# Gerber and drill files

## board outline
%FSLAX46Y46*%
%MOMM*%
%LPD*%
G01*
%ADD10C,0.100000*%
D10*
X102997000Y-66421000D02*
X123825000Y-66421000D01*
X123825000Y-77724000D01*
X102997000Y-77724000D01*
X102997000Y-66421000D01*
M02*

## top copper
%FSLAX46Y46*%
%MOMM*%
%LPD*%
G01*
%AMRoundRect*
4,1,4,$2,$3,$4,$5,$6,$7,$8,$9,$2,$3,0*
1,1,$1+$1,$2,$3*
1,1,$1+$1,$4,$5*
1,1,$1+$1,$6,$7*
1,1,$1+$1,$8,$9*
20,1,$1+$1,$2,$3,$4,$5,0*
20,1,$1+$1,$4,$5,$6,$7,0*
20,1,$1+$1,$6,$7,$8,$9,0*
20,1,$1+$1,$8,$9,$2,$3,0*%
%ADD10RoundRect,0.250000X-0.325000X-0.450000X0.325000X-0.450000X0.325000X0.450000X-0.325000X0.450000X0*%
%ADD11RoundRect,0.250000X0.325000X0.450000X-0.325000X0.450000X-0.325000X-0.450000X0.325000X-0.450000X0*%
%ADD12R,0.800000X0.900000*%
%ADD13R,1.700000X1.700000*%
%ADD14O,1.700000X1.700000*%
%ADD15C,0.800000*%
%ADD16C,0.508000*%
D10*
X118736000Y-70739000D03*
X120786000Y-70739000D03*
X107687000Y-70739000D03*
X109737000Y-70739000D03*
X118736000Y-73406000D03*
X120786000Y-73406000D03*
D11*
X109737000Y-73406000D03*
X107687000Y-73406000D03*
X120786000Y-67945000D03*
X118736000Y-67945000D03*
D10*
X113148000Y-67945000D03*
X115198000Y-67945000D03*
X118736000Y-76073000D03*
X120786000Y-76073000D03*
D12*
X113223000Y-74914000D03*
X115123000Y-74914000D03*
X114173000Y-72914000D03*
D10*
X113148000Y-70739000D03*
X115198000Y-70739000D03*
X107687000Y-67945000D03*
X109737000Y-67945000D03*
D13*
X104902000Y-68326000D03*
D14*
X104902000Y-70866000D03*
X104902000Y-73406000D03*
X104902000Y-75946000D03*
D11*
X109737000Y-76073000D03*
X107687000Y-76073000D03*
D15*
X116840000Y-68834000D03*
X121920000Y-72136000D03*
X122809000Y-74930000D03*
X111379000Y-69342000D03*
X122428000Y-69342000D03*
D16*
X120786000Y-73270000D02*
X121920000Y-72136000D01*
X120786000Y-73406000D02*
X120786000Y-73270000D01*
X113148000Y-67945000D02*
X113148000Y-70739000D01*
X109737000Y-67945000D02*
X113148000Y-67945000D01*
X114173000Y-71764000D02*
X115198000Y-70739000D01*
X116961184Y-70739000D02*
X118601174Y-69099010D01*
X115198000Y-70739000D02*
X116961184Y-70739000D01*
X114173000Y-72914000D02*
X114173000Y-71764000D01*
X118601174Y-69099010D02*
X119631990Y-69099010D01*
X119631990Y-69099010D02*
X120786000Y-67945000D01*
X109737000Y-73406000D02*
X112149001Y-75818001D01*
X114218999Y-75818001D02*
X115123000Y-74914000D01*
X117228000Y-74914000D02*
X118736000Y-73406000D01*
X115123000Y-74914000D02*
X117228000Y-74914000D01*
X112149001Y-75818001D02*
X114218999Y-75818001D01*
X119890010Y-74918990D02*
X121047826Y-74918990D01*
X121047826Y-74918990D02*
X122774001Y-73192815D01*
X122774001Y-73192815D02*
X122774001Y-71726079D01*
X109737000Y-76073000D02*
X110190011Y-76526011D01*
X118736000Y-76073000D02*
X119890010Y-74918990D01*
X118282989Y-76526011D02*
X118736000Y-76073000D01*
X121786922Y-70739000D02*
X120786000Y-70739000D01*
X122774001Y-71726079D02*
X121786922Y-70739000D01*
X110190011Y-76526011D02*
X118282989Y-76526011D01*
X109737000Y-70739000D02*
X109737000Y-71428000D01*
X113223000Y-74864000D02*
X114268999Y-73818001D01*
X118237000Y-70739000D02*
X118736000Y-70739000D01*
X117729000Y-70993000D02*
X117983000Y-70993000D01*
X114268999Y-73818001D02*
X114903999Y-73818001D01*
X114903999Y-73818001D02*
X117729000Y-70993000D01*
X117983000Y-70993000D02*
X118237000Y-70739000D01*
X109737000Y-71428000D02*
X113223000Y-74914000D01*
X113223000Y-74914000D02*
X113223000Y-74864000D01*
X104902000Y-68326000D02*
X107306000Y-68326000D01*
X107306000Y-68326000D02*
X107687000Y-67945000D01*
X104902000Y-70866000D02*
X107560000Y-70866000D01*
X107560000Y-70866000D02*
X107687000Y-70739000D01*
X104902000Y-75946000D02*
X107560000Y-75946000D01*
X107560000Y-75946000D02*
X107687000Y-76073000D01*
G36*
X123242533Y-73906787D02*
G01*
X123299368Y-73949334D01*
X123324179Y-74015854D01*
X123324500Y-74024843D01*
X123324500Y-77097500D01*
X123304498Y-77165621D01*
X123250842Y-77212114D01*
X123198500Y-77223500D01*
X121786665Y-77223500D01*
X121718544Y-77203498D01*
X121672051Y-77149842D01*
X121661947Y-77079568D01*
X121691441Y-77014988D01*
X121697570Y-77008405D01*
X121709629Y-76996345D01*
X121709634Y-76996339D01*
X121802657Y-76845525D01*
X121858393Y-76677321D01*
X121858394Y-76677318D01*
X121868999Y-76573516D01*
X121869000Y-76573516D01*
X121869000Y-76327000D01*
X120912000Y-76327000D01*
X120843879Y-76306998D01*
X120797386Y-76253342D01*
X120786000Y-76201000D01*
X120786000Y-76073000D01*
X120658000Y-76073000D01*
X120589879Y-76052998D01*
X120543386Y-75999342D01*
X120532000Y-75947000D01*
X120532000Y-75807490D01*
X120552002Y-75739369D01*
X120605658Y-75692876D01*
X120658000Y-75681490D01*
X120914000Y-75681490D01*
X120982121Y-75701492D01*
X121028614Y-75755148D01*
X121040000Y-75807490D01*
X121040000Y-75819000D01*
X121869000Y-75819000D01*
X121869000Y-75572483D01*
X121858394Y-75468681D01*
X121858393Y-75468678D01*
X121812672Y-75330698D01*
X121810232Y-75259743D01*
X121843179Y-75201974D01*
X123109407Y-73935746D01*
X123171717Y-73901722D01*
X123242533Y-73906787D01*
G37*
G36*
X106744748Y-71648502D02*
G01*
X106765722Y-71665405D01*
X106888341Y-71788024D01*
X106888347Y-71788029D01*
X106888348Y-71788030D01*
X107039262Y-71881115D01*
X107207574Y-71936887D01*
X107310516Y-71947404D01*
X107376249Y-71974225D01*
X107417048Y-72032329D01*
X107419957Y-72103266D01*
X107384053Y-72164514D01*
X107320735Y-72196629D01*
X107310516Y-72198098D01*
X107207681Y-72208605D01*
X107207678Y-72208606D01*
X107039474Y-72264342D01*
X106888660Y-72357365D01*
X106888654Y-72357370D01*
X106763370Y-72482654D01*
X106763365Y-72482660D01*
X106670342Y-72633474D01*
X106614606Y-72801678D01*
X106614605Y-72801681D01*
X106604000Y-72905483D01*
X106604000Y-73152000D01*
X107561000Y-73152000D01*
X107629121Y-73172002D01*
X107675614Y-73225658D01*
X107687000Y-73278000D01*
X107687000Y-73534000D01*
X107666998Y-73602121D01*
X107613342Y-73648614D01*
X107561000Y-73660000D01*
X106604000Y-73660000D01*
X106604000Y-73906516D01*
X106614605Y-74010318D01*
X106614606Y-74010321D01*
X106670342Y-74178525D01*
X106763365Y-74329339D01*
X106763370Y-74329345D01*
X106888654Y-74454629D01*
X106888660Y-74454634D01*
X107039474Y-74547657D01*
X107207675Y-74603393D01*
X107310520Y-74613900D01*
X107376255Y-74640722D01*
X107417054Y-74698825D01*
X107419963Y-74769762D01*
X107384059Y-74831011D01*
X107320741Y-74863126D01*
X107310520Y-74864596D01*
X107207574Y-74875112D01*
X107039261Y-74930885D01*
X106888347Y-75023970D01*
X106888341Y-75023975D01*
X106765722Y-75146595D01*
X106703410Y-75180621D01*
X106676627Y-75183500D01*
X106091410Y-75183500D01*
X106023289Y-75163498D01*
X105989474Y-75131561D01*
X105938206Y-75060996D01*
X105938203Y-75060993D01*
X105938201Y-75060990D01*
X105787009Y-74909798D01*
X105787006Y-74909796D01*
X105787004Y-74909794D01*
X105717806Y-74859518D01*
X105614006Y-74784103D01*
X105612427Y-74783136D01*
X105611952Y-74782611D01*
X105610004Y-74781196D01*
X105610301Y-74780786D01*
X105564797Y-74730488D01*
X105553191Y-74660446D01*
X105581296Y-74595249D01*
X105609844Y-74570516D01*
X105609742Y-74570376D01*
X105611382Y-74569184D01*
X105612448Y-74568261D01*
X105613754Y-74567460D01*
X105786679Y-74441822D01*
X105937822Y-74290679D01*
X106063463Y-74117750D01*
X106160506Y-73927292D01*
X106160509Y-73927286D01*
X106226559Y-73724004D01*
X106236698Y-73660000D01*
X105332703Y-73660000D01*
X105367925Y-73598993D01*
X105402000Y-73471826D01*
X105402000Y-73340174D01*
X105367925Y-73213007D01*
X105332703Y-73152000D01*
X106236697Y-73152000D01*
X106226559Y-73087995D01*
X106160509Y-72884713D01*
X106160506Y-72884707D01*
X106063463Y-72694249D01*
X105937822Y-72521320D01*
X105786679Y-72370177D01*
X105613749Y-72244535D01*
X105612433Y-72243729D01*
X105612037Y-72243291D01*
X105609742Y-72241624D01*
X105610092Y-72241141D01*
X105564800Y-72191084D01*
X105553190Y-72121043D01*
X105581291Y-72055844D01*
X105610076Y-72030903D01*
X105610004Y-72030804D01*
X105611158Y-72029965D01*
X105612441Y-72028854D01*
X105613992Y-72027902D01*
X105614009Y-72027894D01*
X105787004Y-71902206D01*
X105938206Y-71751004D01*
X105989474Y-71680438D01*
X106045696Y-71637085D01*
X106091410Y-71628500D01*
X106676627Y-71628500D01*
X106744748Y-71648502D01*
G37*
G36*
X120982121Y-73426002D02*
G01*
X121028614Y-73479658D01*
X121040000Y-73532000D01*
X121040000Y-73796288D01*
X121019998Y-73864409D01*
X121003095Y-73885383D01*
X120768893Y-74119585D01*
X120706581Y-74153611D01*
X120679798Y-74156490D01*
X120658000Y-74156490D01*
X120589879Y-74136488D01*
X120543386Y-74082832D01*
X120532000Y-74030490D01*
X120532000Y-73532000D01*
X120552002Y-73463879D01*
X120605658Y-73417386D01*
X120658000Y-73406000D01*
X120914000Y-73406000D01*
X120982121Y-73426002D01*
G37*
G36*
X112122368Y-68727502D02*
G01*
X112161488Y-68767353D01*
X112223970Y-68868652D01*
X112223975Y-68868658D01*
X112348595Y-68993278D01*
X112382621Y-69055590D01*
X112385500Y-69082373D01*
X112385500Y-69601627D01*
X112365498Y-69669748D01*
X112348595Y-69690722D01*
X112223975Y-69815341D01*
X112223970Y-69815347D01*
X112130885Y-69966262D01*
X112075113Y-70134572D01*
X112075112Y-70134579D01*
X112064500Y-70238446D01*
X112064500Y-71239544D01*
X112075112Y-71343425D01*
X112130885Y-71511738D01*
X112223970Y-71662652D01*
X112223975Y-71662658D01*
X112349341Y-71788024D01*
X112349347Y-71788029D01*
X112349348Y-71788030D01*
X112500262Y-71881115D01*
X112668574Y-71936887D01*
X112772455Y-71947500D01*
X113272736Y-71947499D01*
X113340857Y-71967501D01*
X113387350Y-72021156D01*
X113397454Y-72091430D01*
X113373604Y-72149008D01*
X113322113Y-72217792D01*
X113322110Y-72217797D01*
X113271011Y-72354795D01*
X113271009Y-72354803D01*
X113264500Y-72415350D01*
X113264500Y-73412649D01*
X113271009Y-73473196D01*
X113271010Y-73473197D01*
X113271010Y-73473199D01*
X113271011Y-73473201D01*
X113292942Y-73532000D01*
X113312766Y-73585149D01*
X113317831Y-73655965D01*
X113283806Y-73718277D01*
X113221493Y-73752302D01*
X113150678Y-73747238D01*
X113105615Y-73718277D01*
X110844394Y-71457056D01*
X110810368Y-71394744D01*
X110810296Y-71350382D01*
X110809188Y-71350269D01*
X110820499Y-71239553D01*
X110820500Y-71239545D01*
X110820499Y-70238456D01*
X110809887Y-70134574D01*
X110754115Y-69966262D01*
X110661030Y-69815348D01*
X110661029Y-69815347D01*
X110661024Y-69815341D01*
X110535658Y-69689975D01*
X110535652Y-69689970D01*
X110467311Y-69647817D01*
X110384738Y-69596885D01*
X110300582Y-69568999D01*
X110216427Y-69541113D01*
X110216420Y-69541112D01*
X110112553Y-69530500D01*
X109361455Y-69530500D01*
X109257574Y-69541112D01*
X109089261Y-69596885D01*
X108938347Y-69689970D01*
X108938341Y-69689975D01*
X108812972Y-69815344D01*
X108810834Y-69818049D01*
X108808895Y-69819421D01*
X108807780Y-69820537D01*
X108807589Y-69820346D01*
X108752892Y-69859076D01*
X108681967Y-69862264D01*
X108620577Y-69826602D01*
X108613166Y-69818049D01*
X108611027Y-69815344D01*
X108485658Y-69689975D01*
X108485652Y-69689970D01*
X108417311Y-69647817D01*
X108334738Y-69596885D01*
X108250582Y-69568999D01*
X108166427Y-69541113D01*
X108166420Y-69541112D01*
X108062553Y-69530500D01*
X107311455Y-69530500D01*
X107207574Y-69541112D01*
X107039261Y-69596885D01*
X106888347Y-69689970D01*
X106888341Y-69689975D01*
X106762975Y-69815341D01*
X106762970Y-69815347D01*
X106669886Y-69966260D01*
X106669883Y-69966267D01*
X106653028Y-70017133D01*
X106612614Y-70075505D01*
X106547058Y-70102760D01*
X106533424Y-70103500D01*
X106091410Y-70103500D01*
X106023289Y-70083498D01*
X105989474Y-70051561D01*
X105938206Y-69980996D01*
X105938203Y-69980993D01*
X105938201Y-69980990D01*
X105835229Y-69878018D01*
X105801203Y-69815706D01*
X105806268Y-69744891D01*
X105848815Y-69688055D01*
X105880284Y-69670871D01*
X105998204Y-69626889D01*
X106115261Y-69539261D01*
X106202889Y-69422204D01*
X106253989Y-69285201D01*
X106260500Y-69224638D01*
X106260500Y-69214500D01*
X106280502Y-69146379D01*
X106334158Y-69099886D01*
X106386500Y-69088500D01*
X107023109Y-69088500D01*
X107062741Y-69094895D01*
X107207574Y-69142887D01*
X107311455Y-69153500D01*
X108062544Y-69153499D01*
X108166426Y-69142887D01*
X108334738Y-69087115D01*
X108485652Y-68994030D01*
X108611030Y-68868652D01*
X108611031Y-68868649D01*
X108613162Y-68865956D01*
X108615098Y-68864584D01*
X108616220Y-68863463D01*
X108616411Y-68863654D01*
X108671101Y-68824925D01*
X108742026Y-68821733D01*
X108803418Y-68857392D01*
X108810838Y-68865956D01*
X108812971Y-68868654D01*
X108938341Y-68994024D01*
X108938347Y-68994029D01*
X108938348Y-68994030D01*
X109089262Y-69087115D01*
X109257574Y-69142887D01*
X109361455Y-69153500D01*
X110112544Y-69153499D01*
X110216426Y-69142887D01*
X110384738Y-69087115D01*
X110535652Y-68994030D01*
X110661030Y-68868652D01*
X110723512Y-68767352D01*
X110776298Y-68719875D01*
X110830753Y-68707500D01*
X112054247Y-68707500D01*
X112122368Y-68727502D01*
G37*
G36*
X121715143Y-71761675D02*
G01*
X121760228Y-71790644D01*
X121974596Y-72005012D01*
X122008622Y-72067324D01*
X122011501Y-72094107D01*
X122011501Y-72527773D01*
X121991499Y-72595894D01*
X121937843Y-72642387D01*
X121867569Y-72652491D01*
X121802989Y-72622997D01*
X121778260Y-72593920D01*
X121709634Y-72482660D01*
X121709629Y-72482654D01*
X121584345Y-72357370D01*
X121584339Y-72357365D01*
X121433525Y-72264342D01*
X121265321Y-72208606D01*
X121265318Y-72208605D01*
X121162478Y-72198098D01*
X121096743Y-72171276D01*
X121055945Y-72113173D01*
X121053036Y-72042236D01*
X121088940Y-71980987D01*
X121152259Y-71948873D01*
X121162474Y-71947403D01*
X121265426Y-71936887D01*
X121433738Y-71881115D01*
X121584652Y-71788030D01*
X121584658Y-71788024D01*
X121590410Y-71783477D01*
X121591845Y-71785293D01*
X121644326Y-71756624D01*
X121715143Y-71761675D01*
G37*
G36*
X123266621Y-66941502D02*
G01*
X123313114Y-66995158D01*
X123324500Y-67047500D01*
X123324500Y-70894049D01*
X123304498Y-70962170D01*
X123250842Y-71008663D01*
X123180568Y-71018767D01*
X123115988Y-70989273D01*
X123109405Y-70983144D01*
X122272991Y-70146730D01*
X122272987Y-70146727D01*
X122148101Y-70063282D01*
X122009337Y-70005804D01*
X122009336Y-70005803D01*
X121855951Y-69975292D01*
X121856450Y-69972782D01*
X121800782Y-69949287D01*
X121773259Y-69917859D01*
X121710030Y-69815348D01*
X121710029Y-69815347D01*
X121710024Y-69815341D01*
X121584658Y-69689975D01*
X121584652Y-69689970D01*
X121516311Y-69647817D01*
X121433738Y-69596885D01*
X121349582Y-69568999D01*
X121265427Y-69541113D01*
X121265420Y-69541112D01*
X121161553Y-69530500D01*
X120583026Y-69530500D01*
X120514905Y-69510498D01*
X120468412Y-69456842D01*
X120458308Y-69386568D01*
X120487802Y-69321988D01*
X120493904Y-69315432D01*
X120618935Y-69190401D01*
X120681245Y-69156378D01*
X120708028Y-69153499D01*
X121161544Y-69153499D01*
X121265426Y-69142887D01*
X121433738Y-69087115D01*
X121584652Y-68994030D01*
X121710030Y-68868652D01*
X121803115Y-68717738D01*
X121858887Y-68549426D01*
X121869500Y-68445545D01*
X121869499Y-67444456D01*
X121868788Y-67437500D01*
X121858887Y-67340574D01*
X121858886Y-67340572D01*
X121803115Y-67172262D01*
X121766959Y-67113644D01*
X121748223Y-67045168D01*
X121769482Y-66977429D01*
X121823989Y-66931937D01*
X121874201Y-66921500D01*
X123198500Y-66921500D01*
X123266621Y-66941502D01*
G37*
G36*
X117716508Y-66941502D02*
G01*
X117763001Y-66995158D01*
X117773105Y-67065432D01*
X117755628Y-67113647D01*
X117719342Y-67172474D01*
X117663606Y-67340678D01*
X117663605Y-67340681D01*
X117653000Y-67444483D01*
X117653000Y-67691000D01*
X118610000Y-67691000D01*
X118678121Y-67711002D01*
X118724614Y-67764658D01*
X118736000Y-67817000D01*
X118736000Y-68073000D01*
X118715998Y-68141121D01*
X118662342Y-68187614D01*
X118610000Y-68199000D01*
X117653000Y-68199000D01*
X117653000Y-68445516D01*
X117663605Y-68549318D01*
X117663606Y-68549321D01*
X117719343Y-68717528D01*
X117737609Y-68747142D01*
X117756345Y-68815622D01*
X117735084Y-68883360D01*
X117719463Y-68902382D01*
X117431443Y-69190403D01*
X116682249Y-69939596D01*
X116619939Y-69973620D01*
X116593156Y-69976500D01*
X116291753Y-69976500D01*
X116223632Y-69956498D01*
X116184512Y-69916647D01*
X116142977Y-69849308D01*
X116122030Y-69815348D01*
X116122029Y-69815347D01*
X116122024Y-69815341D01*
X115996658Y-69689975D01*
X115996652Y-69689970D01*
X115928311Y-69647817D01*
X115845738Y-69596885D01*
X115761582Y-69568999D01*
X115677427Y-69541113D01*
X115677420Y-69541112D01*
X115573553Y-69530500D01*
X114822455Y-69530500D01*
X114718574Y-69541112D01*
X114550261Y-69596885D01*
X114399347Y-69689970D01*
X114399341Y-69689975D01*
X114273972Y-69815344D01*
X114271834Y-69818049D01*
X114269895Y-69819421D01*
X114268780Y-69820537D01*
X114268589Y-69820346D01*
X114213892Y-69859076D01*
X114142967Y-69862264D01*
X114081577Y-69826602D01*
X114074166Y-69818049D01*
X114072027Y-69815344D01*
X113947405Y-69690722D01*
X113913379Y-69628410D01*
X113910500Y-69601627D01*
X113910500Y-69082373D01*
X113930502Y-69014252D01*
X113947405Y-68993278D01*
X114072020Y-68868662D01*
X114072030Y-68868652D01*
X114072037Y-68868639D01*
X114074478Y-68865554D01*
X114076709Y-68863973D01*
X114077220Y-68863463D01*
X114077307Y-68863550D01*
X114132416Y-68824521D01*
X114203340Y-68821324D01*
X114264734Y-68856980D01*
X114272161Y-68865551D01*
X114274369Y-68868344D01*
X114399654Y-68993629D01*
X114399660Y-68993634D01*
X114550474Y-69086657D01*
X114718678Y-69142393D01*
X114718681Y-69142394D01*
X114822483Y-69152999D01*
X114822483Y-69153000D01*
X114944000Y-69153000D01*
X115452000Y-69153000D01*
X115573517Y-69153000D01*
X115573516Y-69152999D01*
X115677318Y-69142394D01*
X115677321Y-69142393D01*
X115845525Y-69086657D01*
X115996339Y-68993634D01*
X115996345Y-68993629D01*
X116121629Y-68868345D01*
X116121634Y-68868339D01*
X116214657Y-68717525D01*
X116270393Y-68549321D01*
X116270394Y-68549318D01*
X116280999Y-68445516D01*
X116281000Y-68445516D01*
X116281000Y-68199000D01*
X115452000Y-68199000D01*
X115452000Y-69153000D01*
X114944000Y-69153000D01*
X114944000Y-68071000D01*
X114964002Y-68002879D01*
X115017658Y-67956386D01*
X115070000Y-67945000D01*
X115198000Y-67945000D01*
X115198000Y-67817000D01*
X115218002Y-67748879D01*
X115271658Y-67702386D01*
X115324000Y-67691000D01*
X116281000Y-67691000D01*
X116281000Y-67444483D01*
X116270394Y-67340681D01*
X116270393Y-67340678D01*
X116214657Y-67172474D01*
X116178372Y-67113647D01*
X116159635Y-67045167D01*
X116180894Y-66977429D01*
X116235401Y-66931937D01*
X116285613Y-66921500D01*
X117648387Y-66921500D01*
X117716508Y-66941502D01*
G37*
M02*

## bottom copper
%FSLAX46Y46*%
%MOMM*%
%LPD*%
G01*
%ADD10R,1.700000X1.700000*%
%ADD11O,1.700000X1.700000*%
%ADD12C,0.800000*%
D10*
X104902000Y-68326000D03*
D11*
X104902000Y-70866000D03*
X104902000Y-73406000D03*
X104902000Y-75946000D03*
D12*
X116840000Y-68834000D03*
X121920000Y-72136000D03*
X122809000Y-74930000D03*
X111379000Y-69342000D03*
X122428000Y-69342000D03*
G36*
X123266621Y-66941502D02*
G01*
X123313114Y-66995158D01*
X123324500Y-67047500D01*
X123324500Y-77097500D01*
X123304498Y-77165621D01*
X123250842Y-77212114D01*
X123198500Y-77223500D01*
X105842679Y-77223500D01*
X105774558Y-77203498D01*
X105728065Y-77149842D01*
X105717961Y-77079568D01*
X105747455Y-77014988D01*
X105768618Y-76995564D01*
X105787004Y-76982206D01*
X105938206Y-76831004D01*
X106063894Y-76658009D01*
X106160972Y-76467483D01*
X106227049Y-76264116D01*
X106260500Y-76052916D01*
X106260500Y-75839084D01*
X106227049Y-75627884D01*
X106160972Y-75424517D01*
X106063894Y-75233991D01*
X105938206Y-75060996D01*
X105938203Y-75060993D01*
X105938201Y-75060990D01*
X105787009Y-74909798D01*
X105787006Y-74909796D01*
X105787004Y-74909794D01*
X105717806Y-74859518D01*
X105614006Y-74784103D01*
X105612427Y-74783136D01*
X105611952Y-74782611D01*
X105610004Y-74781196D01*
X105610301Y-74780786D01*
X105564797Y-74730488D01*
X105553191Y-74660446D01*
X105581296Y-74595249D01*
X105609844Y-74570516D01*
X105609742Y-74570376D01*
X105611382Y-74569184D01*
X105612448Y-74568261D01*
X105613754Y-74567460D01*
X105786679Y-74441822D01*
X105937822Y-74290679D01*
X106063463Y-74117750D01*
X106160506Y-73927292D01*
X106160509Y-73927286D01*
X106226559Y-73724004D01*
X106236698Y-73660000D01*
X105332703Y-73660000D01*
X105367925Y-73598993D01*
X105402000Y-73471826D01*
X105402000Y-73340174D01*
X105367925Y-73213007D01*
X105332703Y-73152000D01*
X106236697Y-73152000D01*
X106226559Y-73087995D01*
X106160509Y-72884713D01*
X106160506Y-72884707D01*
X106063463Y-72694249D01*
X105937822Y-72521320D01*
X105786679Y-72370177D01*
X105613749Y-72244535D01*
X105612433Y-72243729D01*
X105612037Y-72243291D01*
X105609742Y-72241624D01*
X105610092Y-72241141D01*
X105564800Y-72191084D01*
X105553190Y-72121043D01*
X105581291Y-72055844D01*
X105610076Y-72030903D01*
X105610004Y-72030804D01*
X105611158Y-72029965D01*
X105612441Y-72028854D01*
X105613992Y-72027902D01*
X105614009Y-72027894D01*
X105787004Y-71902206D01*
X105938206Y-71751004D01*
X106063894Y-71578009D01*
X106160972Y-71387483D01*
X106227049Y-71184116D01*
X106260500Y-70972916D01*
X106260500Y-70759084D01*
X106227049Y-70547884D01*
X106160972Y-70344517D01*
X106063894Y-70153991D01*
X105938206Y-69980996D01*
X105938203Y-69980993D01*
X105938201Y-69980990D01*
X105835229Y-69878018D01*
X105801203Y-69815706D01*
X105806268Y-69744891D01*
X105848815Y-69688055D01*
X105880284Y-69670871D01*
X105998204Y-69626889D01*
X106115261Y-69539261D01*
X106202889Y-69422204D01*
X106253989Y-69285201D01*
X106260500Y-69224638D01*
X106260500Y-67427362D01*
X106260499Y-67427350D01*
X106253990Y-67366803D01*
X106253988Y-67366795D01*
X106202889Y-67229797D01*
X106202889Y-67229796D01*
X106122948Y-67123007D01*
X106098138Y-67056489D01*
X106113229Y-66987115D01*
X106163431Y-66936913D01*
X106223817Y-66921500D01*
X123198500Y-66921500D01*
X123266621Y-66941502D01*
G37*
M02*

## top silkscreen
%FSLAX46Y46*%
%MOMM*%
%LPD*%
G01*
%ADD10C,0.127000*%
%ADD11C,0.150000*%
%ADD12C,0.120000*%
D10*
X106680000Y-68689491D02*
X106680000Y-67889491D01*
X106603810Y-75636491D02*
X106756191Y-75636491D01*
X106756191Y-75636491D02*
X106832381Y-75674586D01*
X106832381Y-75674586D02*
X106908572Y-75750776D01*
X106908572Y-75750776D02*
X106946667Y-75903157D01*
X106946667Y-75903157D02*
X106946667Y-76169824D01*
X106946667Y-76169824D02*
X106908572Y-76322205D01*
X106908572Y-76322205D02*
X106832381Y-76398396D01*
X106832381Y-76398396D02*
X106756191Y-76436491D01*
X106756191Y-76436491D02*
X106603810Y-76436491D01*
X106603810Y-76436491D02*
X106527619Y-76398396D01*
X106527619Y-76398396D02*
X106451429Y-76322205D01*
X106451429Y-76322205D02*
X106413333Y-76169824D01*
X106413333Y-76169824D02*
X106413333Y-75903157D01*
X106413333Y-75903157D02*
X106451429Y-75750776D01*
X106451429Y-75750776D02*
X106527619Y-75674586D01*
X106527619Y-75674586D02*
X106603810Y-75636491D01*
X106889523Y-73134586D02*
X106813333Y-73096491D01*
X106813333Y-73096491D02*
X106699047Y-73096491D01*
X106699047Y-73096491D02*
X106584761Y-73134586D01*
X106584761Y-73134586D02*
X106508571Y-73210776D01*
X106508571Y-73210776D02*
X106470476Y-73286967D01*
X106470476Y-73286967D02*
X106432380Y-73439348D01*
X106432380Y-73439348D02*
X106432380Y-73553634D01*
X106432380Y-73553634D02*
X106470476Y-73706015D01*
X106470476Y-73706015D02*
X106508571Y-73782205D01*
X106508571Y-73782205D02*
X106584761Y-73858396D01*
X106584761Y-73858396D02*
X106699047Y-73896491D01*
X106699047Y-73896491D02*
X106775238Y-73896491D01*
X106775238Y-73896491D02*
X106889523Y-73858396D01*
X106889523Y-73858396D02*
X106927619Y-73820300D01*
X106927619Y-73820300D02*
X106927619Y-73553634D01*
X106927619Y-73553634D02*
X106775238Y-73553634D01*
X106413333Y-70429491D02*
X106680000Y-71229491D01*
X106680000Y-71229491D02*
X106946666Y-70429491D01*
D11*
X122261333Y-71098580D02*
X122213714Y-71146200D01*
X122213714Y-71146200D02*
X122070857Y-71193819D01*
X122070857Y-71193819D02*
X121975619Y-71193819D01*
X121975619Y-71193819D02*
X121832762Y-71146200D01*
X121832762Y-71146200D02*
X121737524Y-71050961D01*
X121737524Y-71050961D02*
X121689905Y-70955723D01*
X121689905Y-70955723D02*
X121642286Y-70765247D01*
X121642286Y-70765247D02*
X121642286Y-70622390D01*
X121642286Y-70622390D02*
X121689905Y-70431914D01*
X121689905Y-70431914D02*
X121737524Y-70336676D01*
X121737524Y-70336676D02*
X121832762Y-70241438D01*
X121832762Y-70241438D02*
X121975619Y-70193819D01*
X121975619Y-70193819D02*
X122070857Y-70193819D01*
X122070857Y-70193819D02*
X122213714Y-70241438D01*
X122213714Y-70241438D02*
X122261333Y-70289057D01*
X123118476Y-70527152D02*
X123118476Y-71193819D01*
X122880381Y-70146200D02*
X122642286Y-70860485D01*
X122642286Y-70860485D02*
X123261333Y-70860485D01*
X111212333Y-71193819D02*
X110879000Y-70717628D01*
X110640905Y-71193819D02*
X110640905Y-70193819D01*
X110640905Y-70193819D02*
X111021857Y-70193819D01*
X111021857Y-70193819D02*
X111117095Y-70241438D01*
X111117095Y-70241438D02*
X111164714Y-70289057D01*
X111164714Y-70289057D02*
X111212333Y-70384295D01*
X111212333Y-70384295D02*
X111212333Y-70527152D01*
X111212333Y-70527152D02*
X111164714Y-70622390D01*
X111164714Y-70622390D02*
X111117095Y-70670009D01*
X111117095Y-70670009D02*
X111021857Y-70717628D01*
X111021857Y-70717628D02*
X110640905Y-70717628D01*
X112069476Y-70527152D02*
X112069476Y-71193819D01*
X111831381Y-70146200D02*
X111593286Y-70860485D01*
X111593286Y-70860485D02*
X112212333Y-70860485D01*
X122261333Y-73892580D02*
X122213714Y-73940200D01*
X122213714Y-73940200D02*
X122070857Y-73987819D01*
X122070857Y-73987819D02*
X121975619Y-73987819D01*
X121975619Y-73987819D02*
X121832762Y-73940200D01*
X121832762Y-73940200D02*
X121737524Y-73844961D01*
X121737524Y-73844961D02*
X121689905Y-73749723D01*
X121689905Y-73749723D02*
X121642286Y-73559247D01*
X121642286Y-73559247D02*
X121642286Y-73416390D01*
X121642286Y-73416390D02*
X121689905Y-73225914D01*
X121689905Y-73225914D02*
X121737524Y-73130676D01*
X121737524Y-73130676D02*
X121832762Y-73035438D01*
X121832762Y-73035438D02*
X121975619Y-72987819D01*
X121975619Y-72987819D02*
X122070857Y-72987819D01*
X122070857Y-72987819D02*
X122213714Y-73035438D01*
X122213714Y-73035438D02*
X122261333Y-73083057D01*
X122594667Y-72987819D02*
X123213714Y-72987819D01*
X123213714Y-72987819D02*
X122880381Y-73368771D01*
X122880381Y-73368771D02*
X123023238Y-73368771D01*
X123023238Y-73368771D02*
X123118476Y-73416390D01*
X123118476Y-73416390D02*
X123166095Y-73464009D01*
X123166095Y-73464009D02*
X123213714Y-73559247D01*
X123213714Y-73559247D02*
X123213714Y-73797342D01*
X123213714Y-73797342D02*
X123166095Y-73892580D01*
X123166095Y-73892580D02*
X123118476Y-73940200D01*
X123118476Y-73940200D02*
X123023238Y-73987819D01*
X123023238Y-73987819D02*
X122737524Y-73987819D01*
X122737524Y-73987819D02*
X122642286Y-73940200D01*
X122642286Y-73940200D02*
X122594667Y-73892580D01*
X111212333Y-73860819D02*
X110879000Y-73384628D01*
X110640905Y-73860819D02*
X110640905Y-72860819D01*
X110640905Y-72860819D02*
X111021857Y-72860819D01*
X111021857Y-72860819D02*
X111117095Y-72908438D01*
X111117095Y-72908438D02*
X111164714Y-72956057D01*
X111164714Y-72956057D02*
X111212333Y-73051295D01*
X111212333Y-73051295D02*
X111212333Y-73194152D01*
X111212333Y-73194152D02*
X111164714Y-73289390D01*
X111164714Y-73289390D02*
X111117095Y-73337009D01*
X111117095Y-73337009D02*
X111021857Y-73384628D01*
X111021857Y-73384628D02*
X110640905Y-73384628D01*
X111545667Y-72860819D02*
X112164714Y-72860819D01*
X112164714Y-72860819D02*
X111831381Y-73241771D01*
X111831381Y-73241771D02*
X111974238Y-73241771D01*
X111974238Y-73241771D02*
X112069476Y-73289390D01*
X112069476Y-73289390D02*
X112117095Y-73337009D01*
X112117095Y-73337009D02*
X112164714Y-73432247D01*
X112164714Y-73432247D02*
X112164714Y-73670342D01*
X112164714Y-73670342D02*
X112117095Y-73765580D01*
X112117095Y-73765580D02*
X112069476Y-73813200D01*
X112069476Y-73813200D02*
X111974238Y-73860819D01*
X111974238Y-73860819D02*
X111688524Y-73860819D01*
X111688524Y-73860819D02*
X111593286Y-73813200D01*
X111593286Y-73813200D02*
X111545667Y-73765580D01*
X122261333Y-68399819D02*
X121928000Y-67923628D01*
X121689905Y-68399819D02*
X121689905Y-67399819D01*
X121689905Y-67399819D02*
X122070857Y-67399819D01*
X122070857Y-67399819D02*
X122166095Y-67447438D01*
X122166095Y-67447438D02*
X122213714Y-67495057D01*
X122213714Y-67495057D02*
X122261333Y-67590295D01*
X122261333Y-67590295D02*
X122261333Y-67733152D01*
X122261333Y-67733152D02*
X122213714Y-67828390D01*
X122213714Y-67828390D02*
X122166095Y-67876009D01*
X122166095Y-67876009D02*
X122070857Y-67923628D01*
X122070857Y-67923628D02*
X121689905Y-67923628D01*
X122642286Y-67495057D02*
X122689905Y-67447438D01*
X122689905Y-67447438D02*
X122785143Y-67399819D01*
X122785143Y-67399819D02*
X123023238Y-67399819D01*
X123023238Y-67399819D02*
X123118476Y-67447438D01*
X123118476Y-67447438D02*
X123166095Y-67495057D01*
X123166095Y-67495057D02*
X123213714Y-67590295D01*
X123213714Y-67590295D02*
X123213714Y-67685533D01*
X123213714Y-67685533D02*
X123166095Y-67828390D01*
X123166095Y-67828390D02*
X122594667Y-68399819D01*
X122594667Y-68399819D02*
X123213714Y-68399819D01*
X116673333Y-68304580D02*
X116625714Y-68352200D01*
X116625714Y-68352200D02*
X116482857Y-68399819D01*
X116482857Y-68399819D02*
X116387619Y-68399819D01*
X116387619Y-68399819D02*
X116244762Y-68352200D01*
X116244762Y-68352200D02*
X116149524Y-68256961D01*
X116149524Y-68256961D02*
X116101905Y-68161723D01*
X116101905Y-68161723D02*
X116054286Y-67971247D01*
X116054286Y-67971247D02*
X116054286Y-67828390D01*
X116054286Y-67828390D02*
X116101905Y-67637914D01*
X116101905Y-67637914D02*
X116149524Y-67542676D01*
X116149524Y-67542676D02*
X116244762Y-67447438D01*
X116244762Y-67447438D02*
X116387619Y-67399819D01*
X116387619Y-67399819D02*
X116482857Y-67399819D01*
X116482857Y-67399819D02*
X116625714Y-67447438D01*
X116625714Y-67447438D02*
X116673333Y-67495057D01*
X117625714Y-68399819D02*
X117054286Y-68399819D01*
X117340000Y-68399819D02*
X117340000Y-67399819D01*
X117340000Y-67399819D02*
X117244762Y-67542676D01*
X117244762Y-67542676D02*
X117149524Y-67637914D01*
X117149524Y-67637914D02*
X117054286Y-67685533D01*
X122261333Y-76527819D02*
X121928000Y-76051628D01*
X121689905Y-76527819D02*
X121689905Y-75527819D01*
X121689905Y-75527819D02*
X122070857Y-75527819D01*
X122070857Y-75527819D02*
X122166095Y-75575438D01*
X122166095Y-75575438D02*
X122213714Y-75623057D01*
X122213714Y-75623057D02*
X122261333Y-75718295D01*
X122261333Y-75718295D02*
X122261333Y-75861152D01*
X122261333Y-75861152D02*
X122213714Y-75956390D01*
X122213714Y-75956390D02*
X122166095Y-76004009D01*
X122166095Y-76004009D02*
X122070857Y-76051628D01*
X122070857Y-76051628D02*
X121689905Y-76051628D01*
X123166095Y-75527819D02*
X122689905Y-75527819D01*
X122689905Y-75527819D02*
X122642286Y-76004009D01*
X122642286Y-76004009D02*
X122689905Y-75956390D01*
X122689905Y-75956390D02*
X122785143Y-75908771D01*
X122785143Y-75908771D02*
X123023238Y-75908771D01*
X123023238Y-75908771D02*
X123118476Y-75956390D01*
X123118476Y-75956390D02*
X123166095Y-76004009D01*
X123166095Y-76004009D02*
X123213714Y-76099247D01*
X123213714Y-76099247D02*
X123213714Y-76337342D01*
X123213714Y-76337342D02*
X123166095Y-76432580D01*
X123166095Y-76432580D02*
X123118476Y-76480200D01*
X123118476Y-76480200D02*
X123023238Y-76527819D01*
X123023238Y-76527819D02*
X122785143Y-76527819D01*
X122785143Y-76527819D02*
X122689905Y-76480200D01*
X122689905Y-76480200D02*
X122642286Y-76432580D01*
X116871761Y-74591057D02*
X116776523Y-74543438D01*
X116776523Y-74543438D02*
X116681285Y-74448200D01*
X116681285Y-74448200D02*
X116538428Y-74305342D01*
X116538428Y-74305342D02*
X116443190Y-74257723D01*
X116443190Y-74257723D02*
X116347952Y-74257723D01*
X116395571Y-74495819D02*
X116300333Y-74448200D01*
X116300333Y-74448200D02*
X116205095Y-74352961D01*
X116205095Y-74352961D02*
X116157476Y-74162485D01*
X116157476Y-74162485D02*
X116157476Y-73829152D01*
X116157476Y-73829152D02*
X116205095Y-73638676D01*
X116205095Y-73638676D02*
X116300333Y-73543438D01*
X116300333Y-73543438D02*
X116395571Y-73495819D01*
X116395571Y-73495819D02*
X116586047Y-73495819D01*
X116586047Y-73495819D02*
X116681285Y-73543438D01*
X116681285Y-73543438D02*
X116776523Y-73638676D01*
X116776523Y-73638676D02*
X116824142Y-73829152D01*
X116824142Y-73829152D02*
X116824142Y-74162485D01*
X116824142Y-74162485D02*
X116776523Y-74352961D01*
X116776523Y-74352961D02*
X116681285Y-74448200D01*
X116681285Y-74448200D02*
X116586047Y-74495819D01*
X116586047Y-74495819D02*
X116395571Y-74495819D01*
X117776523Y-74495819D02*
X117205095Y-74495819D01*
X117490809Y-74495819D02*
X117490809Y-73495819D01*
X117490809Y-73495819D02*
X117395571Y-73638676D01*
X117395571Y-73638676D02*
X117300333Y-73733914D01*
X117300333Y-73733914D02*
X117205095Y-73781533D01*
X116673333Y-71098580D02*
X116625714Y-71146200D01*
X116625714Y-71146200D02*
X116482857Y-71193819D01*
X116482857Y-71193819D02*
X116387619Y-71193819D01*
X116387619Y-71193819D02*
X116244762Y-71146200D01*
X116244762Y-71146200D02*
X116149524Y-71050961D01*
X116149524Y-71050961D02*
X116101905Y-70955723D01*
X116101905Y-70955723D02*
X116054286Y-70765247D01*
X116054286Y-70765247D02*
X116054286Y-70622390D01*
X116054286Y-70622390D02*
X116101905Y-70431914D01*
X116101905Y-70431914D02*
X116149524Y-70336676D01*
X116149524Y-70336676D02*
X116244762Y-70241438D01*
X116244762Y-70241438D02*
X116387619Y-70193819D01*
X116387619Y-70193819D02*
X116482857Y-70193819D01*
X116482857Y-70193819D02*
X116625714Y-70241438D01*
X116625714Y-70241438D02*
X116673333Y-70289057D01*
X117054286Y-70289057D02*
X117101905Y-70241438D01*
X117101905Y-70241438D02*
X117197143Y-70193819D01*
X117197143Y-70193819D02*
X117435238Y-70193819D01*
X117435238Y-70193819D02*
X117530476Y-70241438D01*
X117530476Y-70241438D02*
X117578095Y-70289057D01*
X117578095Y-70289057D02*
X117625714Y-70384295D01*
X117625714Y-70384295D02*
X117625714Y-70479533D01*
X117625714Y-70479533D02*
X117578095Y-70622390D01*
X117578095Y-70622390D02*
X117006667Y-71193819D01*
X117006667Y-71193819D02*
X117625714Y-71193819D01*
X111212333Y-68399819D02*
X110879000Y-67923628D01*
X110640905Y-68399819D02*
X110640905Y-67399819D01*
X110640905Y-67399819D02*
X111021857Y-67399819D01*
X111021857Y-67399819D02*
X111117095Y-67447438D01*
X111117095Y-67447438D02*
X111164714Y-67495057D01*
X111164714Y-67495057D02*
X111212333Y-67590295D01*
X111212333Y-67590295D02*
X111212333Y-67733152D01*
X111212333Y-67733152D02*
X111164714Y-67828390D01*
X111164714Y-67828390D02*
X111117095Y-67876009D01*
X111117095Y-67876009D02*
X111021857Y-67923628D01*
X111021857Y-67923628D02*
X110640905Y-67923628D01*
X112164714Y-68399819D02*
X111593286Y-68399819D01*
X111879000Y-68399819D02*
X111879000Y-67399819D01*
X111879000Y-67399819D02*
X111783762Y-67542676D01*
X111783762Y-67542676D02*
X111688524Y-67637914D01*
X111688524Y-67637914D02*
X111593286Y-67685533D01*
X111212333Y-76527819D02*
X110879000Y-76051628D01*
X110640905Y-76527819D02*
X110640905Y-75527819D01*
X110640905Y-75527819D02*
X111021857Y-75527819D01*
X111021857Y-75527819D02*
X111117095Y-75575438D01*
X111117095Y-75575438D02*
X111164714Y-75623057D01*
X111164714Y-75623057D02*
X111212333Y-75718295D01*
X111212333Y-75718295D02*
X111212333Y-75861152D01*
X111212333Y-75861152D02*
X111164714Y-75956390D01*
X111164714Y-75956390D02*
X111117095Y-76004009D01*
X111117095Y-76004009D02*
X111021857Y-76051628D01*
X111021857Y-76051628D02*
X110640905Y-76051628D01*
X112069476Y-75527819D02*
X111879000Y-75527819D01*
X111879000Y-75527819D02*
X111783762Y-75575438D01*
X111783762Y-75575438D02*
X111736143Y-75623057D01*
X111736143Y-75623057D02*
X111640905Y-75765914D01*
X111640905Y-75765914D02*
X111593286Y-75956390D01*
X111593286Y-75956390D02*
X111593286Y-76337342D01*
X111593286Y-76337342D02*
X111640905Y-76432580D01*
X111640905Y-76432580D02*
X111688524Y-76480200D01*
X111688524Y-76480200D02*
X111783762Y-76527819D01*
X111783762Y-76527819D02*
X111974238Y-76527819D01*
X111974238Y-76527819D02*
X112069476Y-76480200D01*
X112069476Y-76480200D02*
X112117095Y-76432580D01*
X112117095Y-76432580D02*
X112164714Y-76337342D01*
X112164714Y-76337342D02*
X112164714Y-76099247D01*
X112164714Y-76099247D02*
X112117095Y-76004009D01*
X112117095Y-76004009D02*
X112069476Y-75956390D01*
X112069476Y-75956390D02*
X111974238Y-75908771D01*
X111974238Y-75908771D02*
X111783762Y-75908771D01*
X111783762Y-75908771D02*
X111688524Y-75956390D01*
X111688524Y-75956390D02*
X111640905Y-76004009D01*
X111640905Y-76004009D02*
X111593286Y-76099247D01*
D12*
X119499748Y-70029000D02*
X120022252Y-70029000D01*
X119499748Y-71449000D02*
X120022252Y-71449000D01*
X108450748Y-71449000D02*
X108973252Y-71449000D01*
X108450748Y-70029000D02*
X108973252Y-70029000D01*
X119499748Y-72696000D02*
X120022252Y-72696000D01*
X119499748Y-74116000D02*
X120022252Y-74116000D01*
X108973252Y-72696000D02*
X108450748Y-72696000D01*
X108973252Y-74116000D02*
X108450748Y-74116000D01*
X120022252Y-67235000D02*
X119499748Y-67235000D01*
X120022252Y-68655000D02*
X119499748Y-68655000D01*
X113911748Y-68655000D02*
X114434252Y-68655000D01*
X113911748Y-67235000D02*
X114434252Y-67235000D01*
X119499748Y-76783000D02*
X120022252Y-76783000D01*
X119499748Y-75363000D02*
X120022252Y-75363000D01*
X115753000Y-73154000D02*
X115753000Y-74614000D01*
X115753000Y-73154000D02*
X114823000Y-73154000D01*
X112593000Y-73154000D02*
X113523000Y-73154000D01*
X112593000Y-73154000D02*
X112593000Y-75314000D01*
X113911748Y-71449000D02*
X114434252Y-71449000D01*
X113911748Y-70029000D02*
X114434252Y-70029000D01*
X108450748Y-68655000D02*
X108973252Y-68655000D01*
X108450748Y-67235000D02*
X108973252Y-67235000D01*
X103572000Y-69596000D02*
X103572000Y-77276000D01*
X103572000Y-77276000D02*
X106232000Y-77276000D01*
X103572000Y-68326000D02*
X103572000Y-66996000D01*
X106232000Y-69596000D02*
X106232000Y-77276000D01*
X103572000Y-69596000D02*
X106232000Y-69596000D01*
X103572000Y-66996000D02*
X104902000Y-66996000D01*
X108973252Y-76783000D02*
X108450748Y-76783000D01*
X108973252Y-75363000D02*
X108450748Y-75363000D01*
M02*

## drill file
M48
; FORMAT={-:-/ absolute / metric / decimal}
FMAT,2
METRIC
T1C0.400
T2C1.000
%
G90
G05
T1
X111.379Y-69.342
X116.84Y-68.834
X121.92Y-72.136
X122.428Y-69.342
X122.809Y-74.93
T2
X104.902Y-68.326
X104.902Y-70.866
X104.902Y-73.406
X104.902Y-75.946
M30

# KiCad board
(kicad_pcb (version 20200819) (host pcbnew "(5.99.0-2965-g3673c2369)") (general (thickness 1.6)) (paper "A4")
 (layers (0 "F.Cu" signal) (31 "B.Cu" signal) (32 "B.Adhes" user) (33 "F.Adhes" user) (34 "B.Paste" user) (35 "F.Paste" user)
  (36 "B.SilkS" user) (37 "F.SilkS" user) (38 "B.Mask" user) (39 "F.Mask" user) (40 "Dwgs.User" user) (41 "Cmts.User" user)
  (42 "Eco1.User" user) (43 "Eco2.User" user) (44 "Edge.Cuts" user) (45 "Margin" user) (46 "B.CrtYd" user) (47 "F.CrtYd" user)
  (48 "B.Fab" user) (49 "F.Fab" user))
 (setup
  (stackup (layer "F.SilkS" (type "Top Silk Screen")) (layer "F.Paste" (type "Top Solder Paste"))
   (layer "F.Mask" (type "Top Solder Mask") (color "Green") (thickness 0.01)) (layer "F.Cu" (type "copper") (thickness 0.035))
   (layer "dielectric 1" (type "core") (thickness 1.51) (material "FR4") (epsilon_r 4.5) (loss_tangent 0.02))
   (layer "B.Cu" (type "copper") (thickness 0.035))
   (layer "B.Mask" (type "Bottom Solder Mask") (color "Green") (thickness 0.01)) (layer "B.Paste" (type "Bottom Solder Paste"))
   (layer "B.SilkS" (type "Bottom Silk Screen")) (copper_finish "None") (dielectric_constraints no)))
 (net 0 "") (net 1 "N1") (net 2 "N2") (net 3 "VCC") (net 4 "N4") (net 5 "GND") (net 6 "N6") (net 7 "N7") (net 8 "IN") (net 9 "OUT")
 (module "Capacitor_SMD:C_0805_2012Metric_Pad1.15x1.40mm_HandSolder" (layer "F.Cu") (at 119.761 70.739)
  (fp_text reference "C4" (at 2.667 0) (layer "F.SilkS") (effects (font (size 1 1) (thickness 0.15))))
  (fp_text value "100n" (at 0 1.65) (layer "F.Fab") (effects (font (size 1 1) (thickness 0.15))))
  (fp_line (start -0.261252 -0.71) (end 0.261252 -0.71) (layer "F.SilkS") (width 0.12))
  (fp_line (start -0.261252 0.71) (end 0.261252 0.71) (layer "F.SilkS") (width 0.12))
  (pad "1" smd roundrect (at -1.025 0) (size 1.15 1.4) (layers "F.Cu" "F.Paste" "F.Mask") (roundrect_rratio 0.2173913043478261) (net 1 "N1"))
  (pad "2" smd roundrect (at 1.025 0) (size 1.15 1.4) (layers "F.Cu" "F.Paste" "F.Mask") (roundrect_rratio 0.2173913043478261) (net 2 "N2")))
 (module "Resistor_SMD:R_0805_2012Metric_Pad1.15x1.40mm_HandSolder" (layer "F.Cu") (at 108.712 70.739)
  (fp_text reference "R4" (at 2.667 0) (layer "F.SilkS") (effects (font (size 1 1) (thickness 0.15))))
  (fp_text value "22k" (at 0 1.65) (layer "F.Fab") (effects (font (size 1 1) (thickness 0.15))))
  (fp_line (start -0.261252 0.71) (end 0.261252 0.71) (layer "F.SilkS") (width 0.12))
  (fp_line (start -0.261252 -0.71) (end 0.261252 -0.71) (layer "F.SilkS") (width 0.12))
  (pad "1" smd roundrect (at -1.025 0) (size 1.15 1.4) (layers "F.Cu" "F.Paste" "F.Mask") (roundrect_rratio 0.2173913043478261)
   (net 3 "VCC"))
  (pad "2" smd roundrect (at 1.025 0) (size 1.15 1.4) (layers "F.Cu" "F.Paste" "F.Mask") (roundrect_rratio 0.2173913043478261) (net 1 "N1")))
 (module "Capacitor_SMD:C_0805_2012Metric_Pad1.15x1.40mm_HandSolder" (layer "F.Cu") (at 119.761 73.406)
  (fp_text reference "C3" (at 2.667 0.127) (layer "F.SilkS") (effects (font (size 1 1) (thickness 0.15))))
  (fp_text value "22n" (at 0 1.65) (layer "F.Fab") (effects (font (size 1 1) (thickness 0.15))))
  (fp_line (start -0.261252 -0.71) (end 0.261252 -0.71) (layer "F.SilkS") (width 0.12))
  (fp_line (start -0.261252 0.71) (end 0.261252 0.71) (layer "F.SilkS") (width 0.12))
  (pad "1" smd roundrect (at -1.025 0) (size 1.15 1.4) (layers "F.Cu" "F.Paste" "F.Mask") (roundrect_rratio 0.2173913043478261) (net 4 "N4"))
  (pad "2" smd roundrect (at 1.025 0) (size 1.15 1.4) (layers "F.Cu" "F.Paste" "F.Mask") (roundrect_rratio 0.2173913043478261) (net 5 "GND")))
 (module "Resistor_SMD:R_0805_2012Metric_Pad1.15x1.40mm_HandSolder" (layer "F.Cu") (at 108.712 73.406 180)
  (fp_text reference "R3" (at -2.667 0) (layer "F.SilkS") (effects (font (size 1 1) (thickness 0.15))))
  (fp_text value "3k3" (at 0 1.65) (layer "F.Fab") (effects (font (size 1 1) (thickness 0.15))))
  (fp_line (start -0.261252 0.71) (end 0.261252 0.71) (layer "F.SilkS") (width 0.12))
  (fp_line (start -0.261252 -0.71) (end 0.261252 -0.71) (layer "F.SilkS") (width 0.12))
  (pad "1" smd roundrect (at -1.025 0 180) (size 1.15 1.4) (layers "F.Cu" "F.Paste" "F.Mask") (roundrect_rratio 0.2173913043478261)
   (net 4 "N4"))
  (pad "2" smd roundrect (at 1.025 0 180) (size 1.15 1.4) (layers "F.Cu" "F.Paste" "F.Mask") (roundrect_rratio 0.2173913043478261)
   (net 5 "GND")))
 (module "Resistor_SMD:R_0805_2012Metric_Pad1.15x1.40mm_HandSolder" (layer "F.Cu") (at 119.761 67.945 180)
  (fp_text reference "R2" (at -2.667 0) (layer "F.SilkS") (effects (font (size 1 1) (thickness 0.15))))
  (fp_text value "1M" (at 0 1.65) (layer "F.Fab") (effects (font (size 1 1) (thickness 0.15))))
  (fp_line (start -0.261252 0.71) (end 0.261252 0.71) (layer "F.SilkS") (width 0.12))
  (fp_line (start -0.261252 -0.71) (end 0.261252 -0.71) (layer "F.SilkS") (width 0.12))
  (pad "1" smd roundrect (at -1.025 0 180) (size 1.15 1.4) (layers "F.Cu" "F.Paste" "F.Mask") (roundrect_rratio 0.2173913043478261)
   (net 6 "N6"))
  (pad "2" smd roundrect (at 1.025 0 180) (size 1.15 1.4) (layers "F.Cu" "F.Paste" "F.Mask") (roundrect_rratio 0.2173913043478261)
   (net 5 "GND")))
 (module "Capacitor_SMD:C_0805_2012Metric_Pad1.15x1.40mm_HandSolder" (layer "F.Cu") (at 114.173 67.945)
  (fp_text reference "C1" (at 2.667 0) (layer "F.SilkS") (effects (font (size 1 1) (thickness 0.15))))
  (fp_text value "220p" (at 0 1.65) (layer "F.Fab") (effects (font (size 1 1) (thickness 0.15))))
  (fp_line (start -0.261252 0.71) (end 0.261252 0.71) (layer "F.SilkS") (width 0.12))
  (fp_line (start -0.261252 -0.71) (end 0.261252 -0.71) (layer "F.SilkS") (width 0.12))
  (pad "1" smd roundrect (at -1.025 0) (size 1.15 1.4) (layers "F.Cu" "F.Paste" "F.Mask") (roundrect_rratio 0.2173913043478261) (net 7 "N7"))
  (pad "2" smd roundrect (at 1.025 0) (size 1.15 1.4) (layers "F.Cu" "F.Paste" "F.Mask") (roundrect_rratio 0.2173913043478261) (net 5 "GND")))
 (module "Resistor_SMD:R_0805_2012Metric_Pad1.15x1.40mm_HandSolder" (layer "F.Cu") (at 119.761 76.073)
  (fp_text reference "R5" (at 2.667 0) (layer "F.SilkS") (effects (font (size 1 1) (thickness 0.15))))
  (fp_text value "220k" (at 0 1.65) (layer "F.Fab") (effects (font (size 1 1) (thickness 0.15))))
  (fp_line (start -0.261252 0.71) (end 0.261252 0.71) (layer "F.SilkS") (width 0.12))
  (fp_line (start -0.261252 -0.71) (end 0.261252 -0.71) (layer "F.SilkS") (width 0.12))
  (pad "1" smd roundrect (at -1.025 0) (size 1.15 1.4) (layers "F.Cu" "F.Paste" "F.Mask") (roundrect_rratio 0.2173913043478261) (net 2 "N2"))
  (pad "2" smd roundrect (at 1.025 0) (size 1.15 1.4) (layers "F.Cu" "F.Paste" "F.Mask") (roundrect_rratio 0.2173913043478261) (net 5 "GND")))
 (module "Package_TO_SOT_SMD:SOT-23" (layer "F.Cu") (at 114.173 73.914 90)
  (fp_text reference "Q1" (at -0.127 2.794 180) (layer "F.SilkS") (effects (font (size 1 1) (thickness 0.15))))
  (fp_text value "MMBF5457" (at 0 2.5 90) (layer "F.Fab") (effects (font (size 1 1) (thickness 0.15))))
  (fp_line (start 0.76 1.58) (end -0.7 1.58) (layer "F.SilkS") (width 0.12))
  (fp_line (start 0.76 1.58) (end 0.76 0.65) (layer "F.SilkS") (width 0.12))
  (fp_line (start 0.76 -1.58) (end 0.76 -0.65) (layer "F.SilkS") (width 0.12))
  (fp_line (start 0.76 -1.58) (end -1.4 -1.58) (layer "F.SilkS") (width 0.12))
  (pad "1" smd rect (at -1 -0.95 90) (size 0.9 0.8) (layers "F.Cu" "F.Paste" "F.Mask") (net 1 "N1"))
  (pad "2" smd rect (at -1 0.95 90) (size 0.9 0.8) (layers "F.Cu" "F.Paste" "F.Mask") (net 4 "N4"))
  (pad "3" smd rect (at 1 0 90) (size 0.9 0.8) (layers "F.Cu" "F.Paste" "F.Mask") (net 6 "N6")))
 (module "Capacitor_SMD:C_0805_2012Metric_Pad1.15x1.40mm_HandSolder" (layer "F.Cu") (at 114.173 70.739)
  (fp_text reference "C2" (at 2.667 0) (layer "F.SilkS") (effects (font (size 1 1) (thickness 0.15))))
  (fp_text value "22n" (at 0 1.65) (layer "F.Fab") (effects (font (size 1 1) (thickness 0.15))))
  (fp_line (start -0.261252 0.71) (end 0.261252 0.71) (layer "F.SilkS") (width 0.12))
  (fp_line (start -0.261252 -0.71) (end 0.261252 -0.71) (layer "F.SilkS") (width 0.12))
  (pad "1" smd roundrect (at -1.025 0) (size 1.15 1.4) (layers "F.Cu" "F.Paste" "F.Mask") (roundrect_rratio 0.2173913043478261) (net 7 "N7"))
  (pad "2" smd roundrect (at 1.025 0) (size 1.15 1.4) (layers "F.Cu" "F.Paste" "F.Mask") (roundrect_rratio 0.2173913043478261) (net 6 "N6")))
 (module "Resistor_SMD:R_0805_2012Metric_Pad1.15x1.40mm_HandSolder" (layer "F.Cu") (at 108.712 67.945)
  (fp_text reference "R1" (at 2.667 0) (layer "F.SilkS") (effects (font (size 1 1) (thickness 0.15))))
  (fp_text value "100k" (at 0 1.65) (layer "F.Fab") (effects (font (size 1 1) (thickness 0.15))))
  (fp_line (start -0.261252 0.71) (end 0.261252 0.71) (layer "F.SilkS") (width 0.12))
  (fp_line (start -0.261252 -0.71) (end 0.261252 -0.71) (layer "F.SilkS") (width 0.12))
  (pad "1" smd roundrect (at -1.025 0) (size 1.15 1.4) (layers "F.Cu" "F.Paste" "F.Mask") (roundrect_rratio 0.2173913043478261) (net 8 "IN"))
  (pad "2" smd roundrect (at 1.025 0) (size 1.15 1.4) (layers "F.Cu" "F.Paste" "F.Mask") (roundrect_rratio 0.2173913043478261) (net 7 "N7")))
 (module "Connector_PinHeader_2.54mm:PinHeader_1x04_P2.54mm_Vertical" (layer "F.Cu") (at 104.902 68.326)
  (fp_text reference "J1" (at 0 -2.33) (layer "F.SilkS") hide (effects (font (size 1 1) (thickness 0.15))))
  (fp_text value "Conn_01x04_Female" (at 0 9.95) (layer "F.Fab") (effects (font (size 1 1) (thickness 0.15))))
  (fp_line (start -1.33 1.27) (end -1.33 8.95) (layer "F.SilkS") (width 0.12))
  (fp_line (start -1.33 8.95) (end 1.33 8.95) (layer "F.SilkS") (width 0.12))
  (fp_line (start -1.33 0) (end -1.33 -1.33) (layer "F.SilkS") (width 0.12))
  (fp_line (start 1.33 1.27) (end 1.33 8.95) (layer "F.SilkS") (width 0.12))
  (fp_line (start -1.33 1.27) (end 1.33 1.27) (layer "F.SilkS") (width 0.12))
  (fp_line (start -1.33 -1.33) (end 0 -1.33) (layer "F.SilkS") (width 0.12))
  (pad "1" thru_hole rect (at 0 0) (size 1.7 1.7) (drill 1) (layers *.Cu *.Mask) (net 8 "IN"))
  (pad "2" thru_hole oval (at 0 2.54) (size 1.7 1.7) (drill 1) (layers *.Cu *.Mask) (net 3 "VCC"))
  (pad "3" thru_hole oval (at 0 5.08) (size 1.7 1.7) (drill 1) (layers *.Cu *.Mask) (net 5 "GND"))
  (pad "4" thru_hole oval (at 0 7.62) (size 1.7 1.7) (drill 1) (layers *.Cu *.Mask) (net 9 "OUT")))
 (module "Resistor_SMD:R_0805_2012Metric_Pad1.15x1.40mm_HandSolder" (layer "F.Cu") (at 108.712 76.073 180)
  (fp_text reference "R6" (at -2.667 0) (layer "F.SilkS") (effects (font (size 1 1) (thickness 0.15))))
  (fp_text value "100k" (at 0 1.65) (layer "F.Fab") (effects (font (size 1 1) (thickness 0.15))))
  (fp_line (start -0.261252 -0.71) (end 0.261252 -0.71) (layer "F.SilkS") (width 0.12))
  (fp_line (start -0.261252 0.71) (end 0.261252 0.71) (layer "F.SilkS") (width 0.12))
  (pad "1" smd roundrect (at -1.025 0 180) (size 1.15 1.4) (layers "F.Cu" "F.Paste" "F.Mask") (roundrect_rratio 0.2173913043478261)
   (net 2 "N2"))
  (pad "2" smd roundrect (at 1.025 0 180) (size 1.15 1.4) (layers "F.Cu" "F.Paste" "F.Mask") (roundrect_rratio 0.2173913043478261)
   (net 9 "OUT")))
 (gr_rect (start 102.997 66.421) (end 123.825 77.724) (layer "Edge.Cuts") (width 0.1))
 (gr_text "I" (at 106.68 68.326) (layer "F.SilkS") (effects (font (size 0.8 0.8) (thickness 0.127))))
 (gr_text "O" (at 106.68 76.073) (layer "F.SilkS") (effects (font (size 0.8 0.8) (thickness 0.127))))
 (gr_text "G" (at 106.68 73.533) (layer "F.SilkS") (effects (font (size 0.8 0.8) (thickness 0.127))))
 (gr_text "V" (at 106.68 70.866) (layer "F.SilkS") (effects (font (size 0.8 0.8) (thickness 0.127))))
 (segment (start 120.786 73.27) (end 121.92 72.136) (width 0.508) (layer "F.Cu") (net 5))
 (segment (start 120.786 73.406) (end 120.786 73.27) (width 0.508) (layer "F.Cu") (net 5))
 (via (at 116.84 68.834) (size 0.8) (drill 0.4) (layers "F.Cu" "B.Cu") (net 5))
 (via (at 121.92 72.136) (size 0.8) (drill 0.4) (layers "F.Cu" "B.Cu") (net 5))
 (via (at 122.809 74.93) (size 0.8) (drill 0.4) (layers "F.Cu" "B.Cu") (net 5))
 (via (at 111.379 69.342) (size 0.8) (drill 0.4) (layers "F.Cu" "B.Cu") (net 5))
 (via (at 122.428 69.342) (size 0.8) (drill 0.4) (layers "F.Cu" "B.Cu") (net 5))
 (segment (start 113.148 67.945) (end 113.148 70.739) (width 0.508) (layer "F.Cu") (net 7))
 (segment (start 109.737 67.945) (end 113.148 67.945) (width 0.508) (layer "F.Cu") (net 7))
 (segment (start 114.173 71.764) (end 115.198 70.739) (width 0.508) (layer "F.Cu") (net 6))
 (segment (start 116.961184 70.739) (end 118.601174 69.09901) (width 0.508) (layer "F.Cu") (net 6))
 (segment (start 115.198 70.739) (end 116.961184 70.739) (width 0.508) (layer "F.Cu") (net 6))
 (segment (start 114.173 72.914) (end 114.173 71.764) (width 0.508) (layer "F.Cu") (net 6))
 (segment (start 118.601174 69.09901) (end 119.63199 69.09901) (width 0.508) (layer "F.Cu") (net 6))
 (segment (start 119.63199 69.09901) (end 120.786 67.945) (width 0.508) (layer "F.Cu") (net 6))
 (segment (start 109.737 73.406) (end 112.149001 75.818001) (width 0.508) (layer "F.Cu") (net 4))
 (segment (start 114.218999 75.818001) (end 115.123 74.914) (width 0.508) (layer "F.Cu") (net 4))
 (segment (start 117.228 74.914) (end 118.736 73.406) (width 0.508) (layer "F.Cu") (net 4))
 (segment (start 115.123 74.914) (end 117.228 74.914) (width 0.508) (layer "F.Cu") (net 4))
 (segment (start 112.149001 75.818001) (end 114.218999 75.818001) (width 0.508) (layer "F.Cu") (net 4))
 (segment (start 119.89001 74.91899) (end 121.047826 74.91899) (width 0.508) (layer "F.Cu") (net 2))
 (segment (start 121.047826 74.91899) (end 122.774001 73.192815) (width 0.508) (layer "F.Cu") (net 2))
 (segment (start 122.774001 73.192815) (end 122.774001 71.726079) (width 0.508) (layer "F.Cu") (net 2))
 (segment (start 109.737 76.073) (end 110.190011 76.526011) (width 0.508) (layer "F.Cu") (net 2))
 (segment (start 118.736 76.073) (end 119.89001 74.91899) (width 0.508) (layer "F.Cu") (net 2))
 (segment (start 118.282989 76.526011) (end 118.736 76.073) (width 0.508) (layer "F.Cu") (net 2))
 (segment (start 121.786922 70.739) (end 120.786 70.739) (width 0.508) (layer "F.Cu") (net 2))
 (segment (start 122.774001 71.726079) (end 121.786922 70.739) (width 0.508) (layer "F.Cu") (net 2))
 (segment (start 110.190011 76.526011) (end 118.282989 76.526011) (width 0.508) (layer "F.Cu") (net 2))
 (segment (start 109.737 70.739) (end 109.737 71.428) (width 0.508) (layer "F.Cu") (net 1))
 (segment (start 113.223 74.864) (end 114.268999 73.818001) (width 0.508) (layer "F.Cu") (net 1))
 (segment (start 118.237 70.739) (end 118.736 70.739) (width 0.508) (layer "F.Cu") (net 1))
 (segment (start 117.729 70.993) (end 117.983 70.993) (width 0.508) (layer "F.Cu") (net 1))
 (segment (start 114.268999 73.818001) (end 114.903999 73.818001) (width 0.508) (layer "F.Cu") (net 1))
 (segment (start 114.903999 73.818001) (end 117.729 70.993) (width 0.508) (layer "F.Cu") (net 1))
 (segment (start 117.983 70.993) (end 118.237 70.739) (width 0.508) (layer "F.Cu") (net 1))
 (segment (start 109.737 71.428) (end 113.223 74.914) (width 0.508) (layer "F.Cu") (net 1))
 (segment (start 113.223 74.914) (end 113.223 74.864) (width 0.508) (layer "F.Cu") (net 1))
 (segment (start 104.902 68.326) (end 107.306 68.326) (width 0.508) (layer "F.Cu") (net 8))
 (segment (start 107.306 68.326) (end 107.687 67.945) (width 0.508) (layer "F.Cu") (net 8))
 (segment (start 104.902 70.866) (end 107.56 70.866) (width 0.508) (layer "F.Cu") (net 3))
 (segment (start 107.56 70.866) (end 107.687 70.739) (width 0.508) (layer "F.Cu") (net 3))
 (segment (start 104.902 75.946) (end 107.56 75.946) (width 0.508) (layer "F.Cu") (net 9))
 (segment (start 107.56 75.946) (end 107.687 76.073) (width 0.508) (layer "F.Cu") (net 9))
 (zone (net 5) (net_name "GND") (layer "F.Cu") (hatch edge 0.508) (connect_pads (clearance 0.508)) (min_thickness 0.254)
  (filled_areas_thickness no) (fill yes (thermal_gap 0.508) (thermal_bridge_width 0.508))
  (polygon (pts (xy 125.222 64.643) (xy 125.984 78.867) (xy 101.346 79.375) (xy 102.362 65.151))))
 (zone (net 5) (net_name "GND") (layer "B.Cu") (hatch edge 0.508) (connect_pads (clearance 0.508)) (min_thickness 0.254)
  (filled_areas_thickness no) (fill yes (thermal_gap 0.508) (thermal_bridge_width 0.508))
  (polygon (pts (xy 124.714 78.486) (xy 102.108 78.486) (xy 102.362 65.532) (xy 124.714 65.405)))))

